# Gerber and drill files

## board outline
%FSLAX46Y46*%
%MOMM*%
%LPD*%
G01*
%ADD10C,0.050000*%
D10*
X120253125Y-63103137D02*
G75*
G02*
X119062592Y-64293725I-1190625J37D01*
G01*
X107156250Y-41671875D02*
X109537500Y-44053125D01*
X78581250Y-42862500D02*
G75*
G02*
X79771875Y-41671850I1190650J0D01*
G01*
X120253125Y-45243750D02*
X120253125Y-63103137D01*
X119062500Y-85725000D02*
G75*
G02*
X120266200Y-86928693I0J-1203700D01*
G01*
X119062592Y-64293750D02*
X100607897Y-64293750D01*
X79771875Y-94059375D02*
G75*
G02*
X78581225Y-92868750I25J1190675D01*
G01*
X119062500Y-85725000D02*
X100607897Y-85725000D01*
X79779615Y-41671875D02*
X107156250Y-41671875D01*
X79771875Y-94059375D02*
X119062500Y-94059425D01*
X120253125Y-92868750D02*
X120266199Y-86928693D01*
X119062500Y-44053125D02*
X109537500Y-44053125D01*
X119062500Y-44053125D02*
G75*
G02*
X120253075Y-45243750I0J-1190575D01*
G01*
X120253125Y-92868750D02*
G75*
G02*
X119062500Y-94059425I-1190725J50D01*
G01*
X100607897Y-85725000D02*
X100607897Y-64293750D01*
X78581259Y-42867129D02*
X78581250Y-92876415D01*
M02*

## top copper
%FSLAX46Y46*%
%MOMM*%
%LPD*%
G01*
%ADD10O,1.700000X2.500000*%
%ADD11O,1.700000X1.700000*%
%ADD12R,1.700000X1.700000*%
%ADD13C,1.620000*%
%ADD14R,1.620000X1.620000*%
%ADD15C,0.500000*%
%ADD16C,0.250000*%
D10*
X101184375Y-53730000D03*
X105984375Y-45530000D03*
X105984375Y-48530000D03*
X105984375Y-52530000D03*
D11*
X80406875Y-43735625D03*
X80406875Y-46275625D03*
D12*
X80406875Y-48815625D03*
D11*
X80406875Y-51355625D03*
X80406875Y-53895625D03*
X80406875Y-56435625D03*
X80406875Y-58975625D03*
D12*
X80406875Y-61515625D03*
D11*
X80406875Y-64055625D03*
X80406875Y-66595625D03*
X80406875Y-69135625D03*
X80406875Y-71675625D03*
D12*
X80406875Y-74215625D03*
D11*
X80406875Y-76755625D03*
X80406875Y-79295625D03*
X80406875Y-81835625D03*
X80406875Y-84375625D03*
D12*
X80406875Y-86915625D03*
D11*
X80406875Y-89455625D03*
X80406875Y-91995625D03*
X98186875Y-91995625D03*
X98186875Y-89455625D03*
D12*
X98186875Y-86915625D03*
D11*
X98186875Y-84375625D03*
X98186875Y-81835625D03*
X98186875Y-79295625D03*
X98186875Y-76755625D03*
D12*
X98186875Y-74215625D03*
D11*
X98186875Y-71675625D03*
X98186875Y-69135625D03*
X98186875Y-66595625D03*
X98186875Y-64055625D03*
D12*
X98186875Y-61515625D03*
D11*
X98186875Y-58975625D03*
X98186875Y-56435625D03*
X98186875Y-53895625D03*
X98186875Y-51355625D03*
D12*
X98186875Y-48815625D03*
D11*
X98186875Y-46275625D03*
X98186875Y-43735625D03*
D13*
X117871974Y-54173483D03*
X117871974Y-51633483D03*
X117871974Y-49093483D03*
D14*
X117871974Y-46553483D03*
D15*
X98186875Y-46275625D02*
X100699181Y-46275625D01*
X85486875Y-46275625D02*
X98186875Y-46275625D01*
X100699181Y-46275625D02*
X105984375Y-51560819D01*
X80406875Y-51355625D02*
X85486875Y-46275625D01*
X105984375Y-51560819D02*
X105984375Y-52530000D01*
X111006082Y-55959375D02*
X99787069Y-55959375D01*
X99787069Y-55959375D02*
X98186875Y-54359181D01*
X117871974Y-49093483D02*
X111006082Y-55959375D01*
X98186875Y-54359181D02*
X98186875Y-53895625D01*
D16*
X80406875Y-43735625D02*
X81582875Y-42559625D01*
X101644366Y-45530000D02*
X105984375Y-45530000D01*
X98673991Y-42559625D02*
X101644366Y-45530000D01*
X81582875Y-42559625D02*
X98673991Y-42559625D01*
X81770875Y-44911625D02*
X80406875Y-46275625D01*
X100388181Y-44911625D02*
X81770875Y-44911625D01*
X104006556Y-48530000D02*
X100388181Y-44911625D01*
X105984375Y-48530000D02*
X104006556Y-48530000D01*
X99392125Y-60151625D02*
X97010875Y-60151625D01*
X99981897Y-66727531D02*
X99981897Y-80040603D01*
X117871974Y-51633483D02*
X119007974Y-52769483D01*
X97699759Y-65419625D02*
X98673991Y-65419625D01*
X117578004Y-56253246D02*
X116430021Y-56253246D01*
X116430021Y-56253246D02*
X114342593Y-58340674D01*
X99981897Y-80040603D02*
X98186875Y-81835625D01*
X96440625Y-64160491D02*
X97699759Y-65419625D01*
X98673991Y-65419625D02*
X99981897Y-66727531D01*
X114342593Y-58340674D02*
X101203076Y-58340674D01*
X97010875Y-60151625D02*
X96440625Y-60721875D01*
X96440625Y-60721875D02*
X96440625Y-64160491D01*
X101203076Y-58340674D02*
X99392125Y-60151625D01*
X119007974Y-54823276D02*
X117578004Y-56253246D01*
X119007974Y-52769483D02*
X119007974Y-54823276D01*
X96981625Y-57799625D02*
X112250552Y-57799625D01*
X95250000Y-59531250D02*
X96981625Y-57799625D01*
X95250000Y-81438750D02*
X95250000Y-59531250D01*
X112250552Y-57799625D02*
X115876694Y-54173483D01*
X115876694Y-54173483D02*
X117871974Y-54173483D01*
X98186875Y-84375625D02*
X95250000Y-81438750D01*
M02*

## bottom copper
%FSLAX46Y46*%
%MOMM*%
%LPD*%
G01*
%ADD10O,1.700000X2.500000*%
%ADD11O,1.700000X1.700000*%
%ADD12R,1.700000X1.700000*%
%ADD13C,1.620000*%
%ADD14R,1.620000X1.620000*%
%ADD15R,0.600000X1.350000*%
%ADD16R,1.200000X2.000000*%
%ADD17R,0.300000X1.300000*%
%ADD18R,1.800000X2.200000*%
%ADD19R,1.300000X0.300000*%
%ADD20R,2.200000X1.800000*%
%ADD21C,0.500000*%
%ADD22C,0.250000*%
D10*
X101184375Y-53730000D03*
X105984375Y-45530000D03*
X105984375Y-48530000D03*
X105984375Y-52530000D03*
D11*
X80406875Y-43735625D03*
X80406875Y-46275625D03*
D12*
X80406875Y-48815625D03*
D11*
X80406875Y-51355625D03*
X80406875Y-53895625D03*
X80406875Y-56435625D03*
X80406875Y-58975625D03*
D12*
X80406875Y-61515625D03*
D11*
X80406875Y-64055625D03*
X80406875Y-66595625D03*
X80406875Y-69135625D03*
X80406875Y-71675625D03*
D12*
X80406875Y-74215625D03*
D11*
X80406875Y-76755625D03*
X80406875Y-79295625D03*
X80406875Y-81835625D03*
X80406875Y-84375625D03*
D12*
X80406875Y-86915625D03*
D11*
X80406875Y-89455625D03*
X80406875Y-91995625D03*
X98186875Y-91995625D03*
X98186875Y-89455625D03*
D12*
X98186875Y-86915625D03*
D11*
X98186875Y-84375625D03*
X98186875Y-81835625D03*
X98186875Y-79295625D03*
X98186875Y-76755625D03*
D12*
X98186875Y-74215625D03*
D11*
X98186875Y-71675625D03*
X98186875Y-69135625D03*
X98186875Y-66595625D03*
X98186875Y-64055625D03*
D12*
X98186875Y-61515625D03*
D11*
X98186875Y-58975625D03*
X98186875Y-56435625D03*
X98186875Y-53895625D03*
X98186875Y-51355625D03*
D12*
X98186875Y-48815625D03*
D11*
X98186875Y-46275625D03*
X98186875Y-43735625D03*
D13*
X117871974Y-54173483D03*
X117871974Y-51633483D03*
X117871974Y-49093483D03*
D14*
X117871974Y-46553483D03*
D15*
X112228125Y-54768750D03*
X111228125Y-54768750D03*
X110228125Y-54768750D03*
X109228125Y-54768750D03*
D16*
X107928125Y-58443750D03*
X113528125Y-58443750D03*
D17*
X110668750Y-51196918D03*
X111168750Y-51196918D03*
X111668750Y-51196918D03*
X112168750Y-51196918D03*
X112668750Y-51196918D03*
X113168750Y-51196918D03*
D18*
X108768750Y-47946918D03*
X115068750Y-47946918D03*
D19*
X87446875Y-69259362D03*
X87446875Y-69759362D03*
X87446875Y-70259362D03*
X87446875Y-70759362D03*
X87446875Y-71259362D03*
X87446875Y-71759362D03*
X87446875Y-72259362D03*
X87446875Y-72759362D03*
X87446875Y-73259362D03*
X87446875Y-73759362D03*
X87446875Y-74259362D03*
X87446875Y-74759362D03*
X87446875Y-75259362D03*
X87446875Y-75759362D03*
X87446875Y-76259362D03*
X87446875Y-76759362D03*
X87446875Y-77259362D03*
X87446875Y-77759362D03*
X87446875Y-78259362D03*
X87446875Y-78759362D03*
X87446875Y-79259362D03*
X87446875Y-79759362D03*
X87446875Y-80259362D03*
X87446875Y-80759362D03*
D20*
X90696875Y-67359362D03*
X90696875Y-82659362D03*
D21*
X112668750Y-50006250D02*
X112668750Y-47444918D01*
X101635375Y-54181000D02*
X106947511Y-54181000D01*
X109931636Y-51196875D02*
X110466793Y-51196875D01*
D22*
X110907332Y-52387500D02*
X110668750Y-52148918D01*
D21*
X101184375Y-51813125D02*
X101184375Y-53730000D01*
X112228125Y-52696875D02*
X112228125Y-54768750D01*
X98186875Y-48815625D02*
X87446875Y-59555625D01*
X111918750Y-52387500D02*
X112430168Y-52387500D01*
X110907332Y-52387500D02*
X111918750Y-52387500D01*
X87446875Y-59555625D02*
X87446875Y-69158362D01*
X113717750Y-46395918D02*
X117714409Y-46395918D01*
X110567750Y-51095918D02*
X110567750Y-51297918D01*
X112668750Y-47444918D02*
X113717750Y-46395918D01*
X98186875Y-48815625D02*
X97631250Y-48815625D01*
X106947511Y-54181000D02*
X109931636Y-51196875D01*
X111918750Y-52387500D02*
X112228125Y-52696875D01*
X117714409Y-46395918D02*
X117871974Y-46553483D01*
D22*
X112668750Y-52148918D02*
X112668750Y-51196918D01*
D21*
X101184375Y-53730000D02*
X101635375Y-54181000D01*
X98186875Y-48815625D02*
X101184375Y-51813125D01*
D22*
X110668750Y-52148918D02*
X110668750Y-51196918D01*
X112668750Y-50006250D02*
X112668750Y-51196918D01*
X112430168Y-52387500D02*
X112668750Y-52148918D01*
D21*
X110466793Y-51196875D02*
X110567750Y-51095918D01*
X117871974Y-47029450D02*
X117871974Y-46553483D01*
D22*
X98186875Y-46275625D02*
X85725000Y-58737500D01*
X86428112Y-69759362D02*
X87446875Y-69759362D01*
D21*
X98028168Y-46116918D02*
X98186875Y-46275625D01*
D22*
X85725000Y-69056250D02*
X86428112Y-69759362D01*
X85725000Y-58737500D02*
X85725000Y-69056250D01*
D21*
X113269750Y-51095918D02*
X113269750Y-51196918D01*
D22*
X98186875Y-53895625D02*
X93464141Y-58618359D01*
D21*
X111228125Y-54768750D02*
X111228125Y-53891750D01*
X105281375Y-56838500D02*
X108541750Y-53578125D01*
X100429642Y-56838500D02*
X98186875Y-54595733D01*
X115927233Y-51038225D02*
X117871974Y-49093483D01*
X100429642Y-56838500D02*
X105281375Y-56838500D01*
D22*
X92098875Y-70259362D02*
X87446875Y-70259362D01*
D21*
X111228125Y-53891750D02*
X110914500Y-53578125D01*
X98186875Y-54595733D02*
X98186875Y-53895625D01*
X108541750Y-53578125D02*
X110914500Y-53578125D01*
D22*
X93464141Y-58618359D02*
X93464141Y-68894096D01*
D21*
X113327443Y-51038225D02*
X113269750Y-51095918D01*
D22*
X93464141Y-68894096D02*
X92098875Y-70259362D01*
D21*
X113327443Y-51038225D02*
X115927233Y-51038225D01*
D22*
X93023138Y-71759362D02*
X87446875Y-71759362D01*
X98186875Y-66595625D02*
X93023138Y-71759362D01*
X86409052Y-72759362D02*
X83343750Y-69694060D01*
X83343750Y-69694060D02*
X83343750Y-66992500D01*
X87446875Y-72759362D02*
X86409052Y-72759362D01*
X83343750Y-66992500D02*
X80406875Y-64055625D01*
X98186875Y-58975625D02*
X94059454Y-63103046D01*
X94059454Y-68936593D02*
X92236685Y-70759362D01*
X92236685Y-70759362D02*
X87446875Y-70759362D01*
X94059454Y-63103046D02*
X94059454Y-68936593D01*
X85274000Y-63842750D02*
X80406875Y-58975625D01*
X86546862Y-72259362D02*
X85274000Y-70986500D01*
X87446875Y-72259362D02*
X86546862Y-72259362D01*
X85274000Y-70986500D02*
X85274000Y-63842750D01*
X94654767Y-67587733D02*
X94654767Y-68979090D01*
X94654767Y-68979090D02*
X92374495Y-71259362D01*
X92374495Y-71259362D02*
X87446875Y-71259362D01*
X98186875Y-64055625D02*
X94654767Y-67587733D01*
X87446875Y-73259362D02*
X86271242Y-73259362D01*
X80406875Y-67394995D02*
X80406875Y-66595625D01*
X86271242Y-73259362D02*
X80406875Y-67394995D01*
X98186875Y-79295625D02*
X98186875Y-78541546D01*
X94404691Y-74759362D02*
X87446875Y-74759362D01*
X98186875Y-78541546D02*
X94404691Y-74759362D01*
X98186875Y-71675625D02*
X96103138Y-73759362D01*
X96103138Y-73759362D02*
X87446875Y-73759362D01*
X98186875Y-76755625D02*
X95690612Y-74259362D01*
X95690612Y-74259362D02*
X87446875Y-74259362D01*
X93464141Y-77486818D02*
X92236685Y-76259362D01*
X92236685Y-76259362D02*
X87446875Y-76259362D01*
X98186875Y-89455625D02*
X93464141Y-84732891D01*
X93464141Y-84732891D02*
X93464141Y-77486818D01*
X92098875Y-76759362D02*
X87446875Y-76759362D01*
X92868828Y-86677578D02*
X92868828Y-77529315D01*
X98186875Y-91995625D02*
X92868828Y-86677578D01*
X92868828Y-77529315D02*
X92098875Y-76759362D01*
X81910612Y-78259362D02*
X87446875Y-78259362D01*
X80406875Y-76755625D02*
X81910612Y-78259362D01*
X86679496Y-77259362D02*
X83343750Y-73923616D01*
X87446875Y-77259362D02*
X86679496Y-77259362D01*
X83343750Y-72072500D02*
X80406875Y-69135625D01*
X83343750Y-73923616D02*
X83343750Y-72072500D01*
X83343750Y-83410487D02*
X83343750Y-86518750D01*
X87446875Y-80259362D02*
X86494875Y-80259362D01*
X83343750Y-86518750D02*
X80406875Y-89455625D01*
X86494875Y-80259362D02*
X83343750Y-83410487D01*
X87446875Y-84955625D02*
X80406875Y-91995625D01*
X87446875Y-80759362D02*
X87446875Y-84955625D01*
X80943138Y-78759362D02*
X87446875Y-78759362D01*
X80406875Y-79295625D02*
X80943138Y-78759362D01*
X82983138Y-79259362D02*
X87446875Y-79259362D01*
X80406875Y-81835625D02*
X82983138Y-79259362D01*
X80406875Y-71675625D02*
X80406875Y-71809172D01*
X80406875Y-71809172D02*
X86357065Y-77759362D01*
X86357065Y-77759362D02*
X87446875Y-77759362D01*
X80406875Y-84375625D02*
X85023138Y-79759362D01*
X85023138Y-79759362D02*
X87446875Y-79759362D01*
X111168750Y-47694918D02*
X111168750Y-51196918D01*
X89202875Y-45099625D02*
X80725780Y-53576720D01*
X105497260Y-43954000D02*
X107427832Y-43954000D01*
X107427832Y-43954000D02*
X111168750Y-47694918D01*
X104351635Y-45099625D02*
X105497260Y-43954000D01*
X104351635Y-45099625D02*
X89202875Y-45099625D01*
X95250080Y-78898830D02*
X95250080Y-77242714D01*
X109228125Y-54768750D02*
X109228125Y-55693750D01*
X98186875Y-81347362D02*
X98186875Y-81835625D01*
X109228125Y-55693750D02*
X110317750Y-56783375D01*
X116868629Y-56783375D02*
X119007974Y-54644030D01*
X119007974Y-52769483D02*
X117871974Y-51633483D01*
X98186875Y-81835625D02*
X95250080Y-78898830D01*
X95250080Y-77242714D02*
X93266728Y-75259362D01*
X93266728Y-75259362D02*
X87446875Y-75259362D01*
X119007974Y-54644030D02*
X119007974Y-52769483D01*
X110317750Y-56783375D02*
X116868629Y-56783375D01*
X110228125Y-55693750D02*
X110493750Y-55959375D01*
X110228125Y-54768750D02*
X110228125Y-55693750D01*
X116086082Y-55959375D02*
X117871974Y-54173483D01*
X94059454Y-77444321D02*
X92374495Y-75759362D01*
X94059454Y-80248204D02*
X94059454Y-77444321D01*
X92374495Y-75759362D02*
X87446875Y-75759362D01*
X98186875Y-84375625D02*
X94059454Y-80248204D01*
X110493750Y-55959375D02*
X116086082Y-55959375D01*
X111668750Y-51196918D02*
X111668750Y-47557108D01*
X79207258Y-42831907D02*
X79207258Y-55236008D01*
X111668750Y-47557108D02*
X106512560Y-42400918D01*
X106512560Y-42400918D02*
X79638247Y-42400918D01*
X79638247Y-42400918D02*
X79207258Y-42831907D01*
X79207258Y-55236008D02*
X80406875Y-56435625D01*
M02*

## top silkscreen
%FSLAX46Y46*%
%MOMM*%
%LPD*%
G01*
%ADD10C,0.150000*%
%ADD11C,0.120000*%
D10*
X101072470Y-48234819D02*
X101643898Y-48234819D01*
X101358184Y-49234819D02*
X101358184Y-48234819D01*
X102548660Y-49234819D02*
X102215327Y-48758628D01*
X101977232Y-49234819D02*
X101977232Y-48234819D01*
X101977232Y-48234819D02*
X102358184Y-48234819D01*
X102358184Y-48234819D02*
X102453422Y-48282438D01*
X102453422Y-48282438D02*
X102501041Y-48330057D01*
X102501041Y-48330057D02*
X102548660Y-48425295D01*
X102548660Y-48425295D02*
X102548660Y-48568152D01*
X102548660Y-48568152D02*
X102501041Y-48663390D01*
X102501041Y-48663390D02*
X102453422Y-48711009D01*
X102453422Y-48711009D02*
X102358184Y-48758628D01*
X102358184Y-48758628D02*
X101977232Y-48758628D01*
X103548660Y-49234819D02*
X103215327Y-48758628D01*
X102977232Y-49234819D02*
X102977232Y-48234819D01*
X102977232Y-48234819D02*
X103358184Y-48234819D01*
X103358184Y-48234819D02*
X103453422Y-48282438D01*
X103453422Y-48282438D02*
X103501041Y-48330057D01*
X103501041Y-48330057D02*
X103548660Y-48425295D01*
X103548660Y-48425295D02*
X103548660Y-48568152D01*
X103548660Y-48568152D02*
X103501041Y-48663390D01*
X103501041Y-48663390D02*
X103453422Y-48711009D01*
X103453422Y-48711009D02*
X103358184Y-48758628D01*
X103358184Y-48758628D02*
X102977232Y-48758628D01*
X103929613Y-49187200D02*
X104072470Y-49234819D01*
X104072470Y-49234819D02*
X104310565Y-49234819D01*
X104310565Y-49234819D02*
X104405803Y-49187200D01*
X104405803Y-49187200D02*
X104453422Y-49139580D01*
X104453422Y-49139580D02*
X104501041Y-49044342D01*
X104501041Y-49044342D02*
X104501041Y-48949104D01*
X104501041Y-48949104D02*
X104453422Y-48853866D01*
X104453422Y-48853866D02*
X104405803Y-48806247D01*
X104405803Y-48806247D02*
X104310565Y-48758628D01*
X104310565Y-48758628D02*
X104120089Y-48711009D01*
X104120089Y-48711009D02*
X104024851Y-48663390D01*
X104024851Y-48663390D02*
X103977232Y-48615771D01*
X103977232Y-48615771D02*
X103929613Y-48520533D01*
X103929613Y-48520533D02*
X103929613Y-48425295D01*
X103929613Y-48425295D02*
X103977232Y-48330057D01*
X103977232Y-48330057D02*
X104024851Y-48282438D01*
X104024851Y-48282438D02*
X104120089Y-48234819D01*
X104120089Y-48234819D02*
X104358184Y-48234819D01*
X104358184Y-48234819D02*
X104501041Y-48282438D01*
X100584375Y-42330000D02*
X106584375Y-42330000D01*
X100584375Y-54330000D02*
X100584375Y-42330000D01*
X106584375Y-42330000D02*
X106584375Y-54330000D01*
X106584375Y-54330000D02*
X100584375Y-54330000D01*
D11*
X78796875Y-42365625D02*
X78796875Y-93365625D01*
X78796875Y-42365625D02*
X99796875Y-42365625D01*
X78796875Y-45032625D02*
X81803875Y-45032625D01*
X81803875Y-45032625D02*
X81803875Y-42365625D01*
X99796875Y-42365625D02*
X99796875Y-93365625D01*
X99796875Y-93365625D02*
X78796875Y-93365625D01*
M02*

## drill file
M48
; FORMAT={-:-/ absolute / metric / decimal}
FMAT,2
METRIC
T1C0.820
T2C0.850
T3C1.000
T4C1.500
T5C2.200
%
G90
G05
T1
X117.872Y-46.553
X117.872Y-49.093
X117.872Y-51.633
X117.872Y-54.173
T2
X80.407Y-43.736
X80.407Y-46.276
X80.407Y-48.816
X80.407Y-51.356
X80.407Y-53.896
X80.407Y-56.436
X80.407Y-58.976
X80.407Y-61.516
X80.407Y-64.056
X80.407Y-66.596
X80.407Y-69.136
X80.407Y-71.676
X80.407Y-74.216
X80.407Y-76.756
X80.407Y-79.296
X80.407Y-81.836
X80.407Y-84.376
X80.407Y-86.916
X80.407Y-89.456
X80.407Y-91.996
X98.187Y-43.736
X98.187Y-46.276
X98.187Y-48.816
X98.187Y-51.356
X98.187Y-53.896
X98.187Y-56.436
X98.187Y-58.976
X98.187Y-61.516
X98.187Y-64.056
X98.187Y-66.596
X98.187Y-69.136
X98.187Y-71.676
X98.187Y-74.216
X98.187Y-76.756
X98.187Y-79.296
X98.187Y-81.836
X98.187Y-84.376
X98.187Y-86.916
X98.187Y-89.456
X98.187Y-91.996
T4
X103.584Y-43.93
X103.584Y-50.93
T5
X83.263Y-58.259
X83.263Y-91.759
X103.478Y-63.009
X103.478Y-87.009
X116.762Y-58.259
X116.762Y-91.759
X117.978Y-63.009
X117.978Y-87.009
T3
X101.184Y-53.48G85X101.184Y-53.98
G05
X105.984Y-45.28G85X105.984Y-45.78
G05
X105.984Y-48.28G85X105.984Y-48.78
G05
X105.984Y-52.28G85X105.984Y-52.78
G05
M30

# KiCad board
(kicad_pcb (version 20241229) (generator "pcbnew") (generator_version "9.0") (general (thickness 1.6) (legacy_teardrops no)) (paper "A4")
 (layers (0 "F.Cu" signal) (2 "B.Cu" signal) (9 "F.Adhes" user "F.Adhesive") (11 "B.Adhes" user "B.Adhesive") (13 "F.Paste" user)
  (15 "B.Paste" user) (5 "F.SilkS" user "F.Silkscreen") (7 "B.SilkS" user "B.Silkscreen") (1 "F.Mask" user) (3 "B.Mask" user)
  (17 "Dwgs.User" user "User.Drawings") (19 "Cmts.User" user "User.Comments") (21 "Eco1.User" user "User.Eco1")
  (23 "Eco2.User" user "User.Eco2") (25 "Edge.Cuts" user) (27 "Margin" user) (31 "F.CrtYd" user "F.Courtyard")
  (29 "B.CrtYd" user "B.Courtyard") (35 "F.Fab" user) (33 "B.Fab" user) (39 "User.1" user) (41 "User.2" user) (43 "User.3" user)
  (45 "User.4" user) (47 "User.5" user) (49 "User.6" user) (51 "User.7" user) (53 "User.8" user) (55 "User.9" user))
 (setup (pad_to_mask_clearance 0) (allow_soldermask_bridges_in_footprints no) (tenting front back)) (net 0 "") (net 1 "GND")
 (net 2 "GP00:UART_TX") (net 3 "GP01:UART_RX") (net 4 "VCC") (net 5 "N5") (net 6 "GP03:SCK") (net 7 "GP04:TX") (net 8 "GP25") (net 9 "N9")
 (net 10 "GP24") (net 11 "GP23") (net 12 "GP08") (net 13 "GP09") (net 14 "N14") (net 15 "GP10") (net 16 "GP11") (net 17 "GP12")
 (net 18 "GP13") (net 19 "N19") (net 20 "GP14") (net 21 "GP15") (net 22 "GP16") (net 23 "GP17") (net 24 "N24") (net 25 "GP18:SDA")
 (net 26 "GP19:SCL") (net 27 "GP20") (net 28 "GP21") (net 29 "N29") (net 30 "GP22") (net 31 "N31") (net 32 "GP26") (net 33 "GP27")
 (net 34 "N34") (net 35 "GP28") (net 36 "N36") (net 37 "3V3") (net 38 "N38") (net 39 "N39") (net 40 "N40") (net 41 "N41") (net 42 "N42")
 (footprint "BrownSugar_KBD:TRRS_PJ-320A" (layer "F.Cu") (at 103.584375 42.33)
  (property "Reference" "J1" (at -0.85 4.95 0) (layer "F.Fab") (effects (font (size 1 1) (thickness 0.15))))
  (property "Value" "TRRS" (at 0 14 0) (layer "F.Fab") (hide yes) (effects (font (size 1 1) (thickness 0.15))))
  (fp_line (start -3 0) (end 3 0) (stroke (width 0.15) (type solid)) (layer "F.SilkS"))
  (fp_line (start -3 12) (end -3 0) (stroke (width 0.15) (type solid)) (layer "F.SilkS"))
  (fp_line (start 3 0) (end 3 12) (stroke (width 0.15) (type solid)) (layer "F.SilkS"))
  (fp_line (start 3 12) (end -3 12) (stroke (width 0.15) (type solid)) (layer "F.SilkS"))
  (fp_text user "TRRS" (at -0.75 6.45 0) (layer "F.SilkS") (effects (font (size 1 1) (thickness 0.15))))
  (pad "" np_thru_hole circle (at 0 1.6) (size 1.5 1.5) (drill 1.5) (layers "*.Cu" "*.Mask"))
  (pad "" np_thru_hole circle (at 0 8.6) (size 1.5 1.5) (drill 1.5) (layers "*.Cu" "*.Mask"))
  (pad "A" thru_hole oval (at -2.4 11.4) (size 1.7 2.5) (drill oval 1 1.5) (layers "*.Cu" "*.Mask") (remove_unused_layers no) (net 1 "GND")
   (clearance 0.15))
  (pad "B" thru_hole oval (at 2.4 3.2) (size 1.7 2.5) (drill oval 1 1.5) (layers "*.Cu" "*.Mask") (remove_unused_layers no)
   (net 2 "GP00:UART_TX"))
  (pad "C" thru_hole oval (at 2.4 6.2) (size 1.7 2.5) (drill oval 1 1.5) (layers "*.Cu" "*.Mask") (remove_unused_layers no)
   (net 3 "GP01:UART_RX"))
  (pad "D" thru_hole oval (at 2.4 10.2) (size 1.7 2.5) (drill oval 1 1.5) (layers "*.Cu" "*.Mask") (remove_unused_layers no) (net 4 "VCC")
   (clearance 0.15)))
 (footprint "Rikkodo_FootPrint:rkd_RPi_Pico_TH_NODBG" (layer "F.Cu") (at 89.296875 67.865625)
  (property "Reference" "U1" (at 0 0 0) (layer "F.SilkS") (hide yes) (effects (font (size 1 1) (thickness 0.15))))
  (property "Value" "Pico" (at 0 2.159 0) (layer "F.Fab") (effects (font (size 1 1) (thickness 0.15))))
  (fp_line (start -10.5 -25.5) (end -10.5 25.5) (stroke (width 0.12) (type solid)) (layer "F.SilkS"))
  (fp_line (start -10.5 -25.5) (end 10.5 -25.5) (stroke (width 0.12) (type solid)) (layer "F.SilkS"))
  (fp_line (start -10.5 -22.833) (end -7.493 -22.833) (stroke (width 0.12) (type solid)) (layer "F.SilkS"))
  (fp_line (start -7.493 -22.833) (end -7.493 -25.5) (stroke (width 0.12) (type solid)) (layer "F.SilkS"))
  (fp_line (start 10.5 -25.5) (end 10.5 25.5) (stroke (width 0.12) (type solid)) (layer "F.SilkS"))
  (fp_line (start 10.5 25.5) (end -10.5 25.5) (stroke (width 0.12) (type solid)) (layer "F.SilkS"))
  (pad "1" thru_hole oval (at -8.89 -24.13) (size 1.7 1.7) (drill 0.85) (layers "*.Cu" "*.Mask") (remove_unused_layers no)
   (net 2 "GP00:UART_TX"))
  (pad "2" thru_hole oval (at -8.89 -21.59) (size 1.7 1.7) (drill 0.85) (layers "*.Cu" "*.Mask") (remove_unused_layers no)
   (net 3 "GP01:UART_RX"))
  (pad "3" thru_hole rect (at -8.89 -19.05) (size 1.7 1.7) (drill 0.85) (layers "*.Cu" "*.Mask") (remove_unused_layers no) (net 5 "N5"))
  (pad "4" thru_hole oval (at -8.89 -16.51) (size 1.7 1.7) (drill 0.85) (layers "*.Cu" "*.Mask") (remove_unused_layers no) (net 4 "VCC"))
  (pad "5" thru_hole oval (at -8.89 -13.97) (size 1.7 1.7) (drill 0.85) (layers "*.Cu" "*.Mask") (remove_unused_layers no)
   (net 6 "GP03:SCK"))
  (pad "6" thru_hole oval (at -8.89 -11.43) (size 1.7 1.7) (drill 0.85) (layers "*.Cu" "*.Mask") (remove_unused_layers no) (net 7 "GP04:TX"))
  (pad "7" thru_hole oval (at -8.89 -8.89) (size 1.7 1.7) (drill 0.85) (layers "*.Cu" "*.Mask") (remove_unused_layers no) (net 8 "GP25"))
  (pad "8" thru_hole rect (at -8.89 -6.35) (size 1.7 1.7) (drill 0.85) (layers "*.Cu" "*.Mask") (remove_unused_layers no) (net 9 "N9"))
  (pad "9" thru_hole oval (at -8.89 -3.81) (size 1.7 1.7) (drill 0.85) (layers "*.Cu" "*.Mask") (remove_unused_layers no) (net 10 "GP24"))
  (pad "10" thru_hole oval (at -8.89 -1.27) (size 1.7 1.7) (drill 0.85) (layers "*.Cu" "*.Mask") (remove_unused_layers no) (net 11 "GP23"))
  (pad "11" thru_hole oval (at -8.89 1.27) (size 1.7 1.7) (drill 0.85) (layers "*.Cu" "*.Mask") (remove_unused_layers no) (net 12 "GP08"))
  (pad "12" thru_hole oval (at -8.89 3.81) (size 1.7 1.7) (drill 0.85) (layers "*.Cu" "*.Mask") (remove_unused_layers no) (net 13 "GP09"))
  (pad "13" thru_hole rect (at -8.89 6.35) (size 1.7 1.7) (drill 0.85) (layers "*.Cu" "*.Mask") (remove_unused_layers no) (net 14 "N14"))
  (pad "14" thru_hole oval (at -8.89 8.89) (size 1.7 1.7) (drill 0.85) (layers "*.Cu" "*.Mask") (remove_unused_layers no) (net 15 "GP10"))
  (pad "15" thru_hole oval (at -8.89 11.43) (size 1.7 1.7) (drill 0.85) (layers "*.Cu" "*.Mask") (remove_unused_layers no) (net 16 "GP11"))
  (pad "16" thru_hole oval (at -8.89 13.97) (size 1.7 1.7) (drill 0.85) (layers "*.Cu" "*.Mask") (remove_unused_layers no) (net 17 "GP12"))
  (pad "17" thru_hole oval (at -8.89 16.51) (size 1.7 1.7) (drill 0.85) (layers "*.Cu" "*.Mask") (remove_unused_layers no) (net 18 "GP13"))
  (pad "18" thru_hole rect (at -8.89 19.05) (size 1.7 1.7) (drill 0.85) (layers "*.Cu" "*.Mask") (remove_unused_layers no) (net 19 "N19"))
  (pad "19" thru_hole oval (at -8.89 21.59) (size 1.7 1.7) (drill 0.85) (layers "*.Cu" "*.Mask") (remove_unused_layers no) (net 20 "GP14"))
  (pad "20" thru_hole oval (at -8.89 24.13) (size 1.7 1.7) (drill 0.85) (layers "*.Cu" "*.Mask") (remove_unused_layers no) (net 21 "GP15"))
  (pad "21" thru_hole oval (at 8.89 24.13) (size 1.7 1.7) (drill 0.85) (layers "*.Cu" "*.Mask") (remove_unused_layers no) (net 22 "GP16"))
  (pad "22" thru_hole oval (at 8.89 21.59) (size 1.7 1.7) (drill 0.85) (layers "*.Cu" "*.Mask") (remove_unused_layers no) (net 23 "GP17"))
  (pad "23" thru_hole rect (at 8.89 19.05) (size 1.7 1.7) (drill 0.85) (layers "*.Cu" "*.Mask") (remove_unused_layers no) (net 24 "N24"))
  (pad "24" thru_hole oval (at 8.89 16.51) (size 1.7 1.7) (drill 0.85) (layers "*.Cu" "*.Mask") (remove_unused_layers no)
   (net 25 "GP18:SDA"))
  (pad "25" thru_hole oval (at 8.89 13.97) (size 1.7 1.7) (drill 0.85) (layers "*.Cu" "*.Mask") (remove_unused_layers no)
   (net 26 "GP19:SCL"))
  (pad "26" thru_hole oval (at 8.89 11.43) (size 1.7 1.7) (drill 0.85) (layers "*.Cu" "*.Mask") (remove_unused_layers no) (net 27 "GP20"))
  (pad "27" thru_hole oval (at 8.89 8.89) (size 1.7 1.7) (drill 0.85) (layers "*.Cu" "*.Mask") (remove_unused_layers no) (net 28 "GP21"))
  (pad "28" thru_hole rect (at 8.89 6.35) (size 1.7 1.7) (drill 0.85) (layers "*.Cu" "*.Mask") (remove_unused_layers no) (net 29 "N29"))
  (pad "29" thru_hole oval (at 8.89 3.81) (size 1.7 1.7) (drill 0.85) (layers "*.Cu" "*.Mask") (remove_unused_layers no) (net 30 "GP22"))
  (pad "30" thru_hole oval (at 8.89 1.27) (size 1.7 1.7) (drill 0.85) (layers "*.Cu" "*.Mask") (remove_unused_layers no) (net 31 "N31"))
  (pad "31" thru_hole oval (at 8.89 -1.27) (size 1.7 1.7) (drill 0.85) (layers "*.Cu" "*.Mask") (remove_unused_layers no) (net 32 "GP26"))
  (pad "32" thru_hole oval (at 8.89 -3.81) (size 1.7 1.7) (drill 0.85) (layers "*.Cu" "*.Mask") (remove_unused_layers no) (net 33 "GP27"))
  (pad "33" thru_hole rect (at 8.89 -6.35) (size 1.7 1.7) (drill 0.85) (layers "*.Cu" "*.Mask") (remove_unused_layers no) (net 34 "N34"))
  (pad "34" thru_hole oval (at 8.89 -8.89) (size 1.7 1.7) (drill 0.85) (layers "*.Cu" "*.Mask") (remove_unused_layers no) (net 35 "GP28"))
  (pad "35" thru_hole oval (at 8.89 -11.43) (size 1.7 1.7) (drill 0.85) (layers "*.Cu" "*.Mask") (remove_unused_layers no) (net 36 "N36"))
  (pad "36" thru_hole oval (at 8.89 -13.97) (size 1.7 1.7) (drill 0.85) (layers "*.Cu" "*.Mask") (remove_unused_layers no) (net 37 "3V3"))
  (pad "37" thru_hole oval (at 8.89 -16.51) (size 1.7 1.7) (drill 0.85) (layers "*.Cu" "*.Mask") (remove_unused_layers no) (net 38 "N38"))
  (pad "38" thru_hole rect (at 8.89 -19.05) (size 1.7 1.7) (drill 0.85) (layers "*.Cu" "*.Mask") (remove_unused_layers no) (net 1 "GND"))
  (pad "39" thru_hole oval (at 8.89 -21.59) (size 1.7 1.7) (drill 0.85) (layers "*.Cu" "*.Mask") (remove_unused_layers no) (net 4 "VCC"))
  (pad "40" thru_hole oval (at 8.89 -24.13) (size 1.7 1.7) (drill 0.85) (layers "*.Cu" "*.Mask") (remove_unused_layers no) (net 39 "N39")))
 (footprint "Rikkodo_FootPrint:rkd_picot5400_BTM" (layer "F.Cu") (at 100.0125 75.009375)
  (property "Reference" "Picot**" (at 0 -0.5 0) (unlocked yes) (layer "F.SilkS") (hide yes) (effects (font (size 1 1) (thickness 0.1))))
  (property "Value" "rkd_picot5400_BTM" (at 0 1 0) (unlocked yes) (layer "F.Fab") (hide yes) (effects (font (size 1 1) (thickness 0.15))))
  (pad "" np_thru_hole circle (at -16.75 -16.75) (size 2.2 2.2) (drill 2.2) (layers "*.Cu" "*.Mask"))
  (pad "" np_thru_hole circle (at -16.75 16.75) (size 2.2 2.2) (drill 2.2) (layers "*.Cu" "*.Mask"))
  (pad "" np_thru_hole circle (at 16.75 -16.75) (size 2.2 2.2) (drill 2.2) (layers "*.Cu" "*.Mask"))
  (pad "" np_thru_hole circle (at 16.75 16.75) (size 2.2 2.2) (drill 2.2) (layers "*.Cu" "*.Mask")))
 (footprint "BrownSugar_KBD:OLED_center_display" (layer "F.Cu") (at 99.371974 50.363483 90)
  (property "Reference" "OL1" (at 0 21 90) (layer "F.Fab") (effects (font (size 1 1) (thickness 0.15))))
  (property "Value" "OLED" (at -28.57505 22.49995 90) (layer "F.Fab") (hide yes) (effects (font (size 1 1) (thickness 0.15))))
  (pad "1" thru_hole circle (at -3.81 18.5 90) (size 1.62 1.62) (drill 0.82) (layers "*.Cu" "*.Mask") (remove_unused_layers no)
   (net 25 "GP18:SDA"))
  (pad "2" thru_hole circle (at -1.27 18.5 90) (size 1.62 1.62) (drill 0.82) (layers "*.Cu" "*.Mask") (remove_unused_layers no)
   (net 26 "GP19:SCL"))
  (pad "3" thru_hole circle (at 1.27 18.5 90) (size 1.62 1.62) (drill 0.82) (layers "*.Cu" "*.Mask") (remove_unused_layers no)
   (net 37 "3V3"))
  (pad "4" thru_hole rect (at 3.81 18.5 90) (size 1.62 1.62) (drill 0.82) (layers "*.Cu" "*.Mask") (remove_unused_layers no) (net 1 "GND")))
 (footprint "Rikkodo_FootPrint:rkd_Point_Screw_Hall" (layer "F.Cu") (at 110.728125 75.009375)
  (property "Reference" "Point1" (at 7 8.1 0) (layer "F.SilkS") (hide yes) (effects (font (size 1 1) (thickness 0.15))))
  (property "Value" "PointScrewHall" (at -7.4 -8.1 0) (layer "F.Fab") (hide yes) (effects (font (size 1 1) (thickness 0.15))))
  (pad "" np_thru_hole circle (at -7.25 -12) (size 2.2 2.2) (drill 2.2) (layers "*.Cu" "*.Mask"))
  (pad "" np_thru_hole circle (at -7.25 12) (size 2.2 2.2) (drill 2.2) (layers "*.Cu" "*.Mask"))
  (pad "" np_thru_hole circle (at 7.25 -12) (size 2.2 2.2) (drill 2.2) (layers "*.Cu" "*.Mask"))
  (pad "" np_thru_hole circle (at 7.25 12) (size 2.2 2.2) (drill 2.2) (layers "*.Cu" "*.Mask")))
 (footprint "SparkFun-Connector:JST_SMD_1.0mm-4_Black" (layer "B.Cu") (at 110.728125 54.76875 180)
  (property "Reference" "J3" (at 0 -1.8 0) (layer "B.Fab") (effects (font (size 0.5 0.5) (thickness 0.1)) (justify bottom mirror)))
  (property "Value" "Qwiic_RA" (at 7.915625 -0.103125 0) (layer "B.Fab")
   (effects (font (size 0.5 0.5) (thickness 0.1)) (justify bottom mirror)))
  (pad "1" smd rect (at -1.5 0 180) (size 0.6 1.35) (layers "B.Cu" "B.Mask" "B.Paste") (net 1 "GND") (thermal_bridge_angle 0))
  (pad "2" smd rect (at -0.5 0 180) (size 0.6 1.35) (layers "B.Cu" "B.Mask" "B.Paste") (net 37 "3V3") (thermal_bridge_angle 0))
  (pad "3" smd rect (at 0.5 0 180) (size 0.6 1.35) (layers "B.Cu" "B.Mask" "B.Paste") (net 25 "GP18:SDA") (thermal_bridge_angle 0))
  (pad "4" smd rect (at 1.5 0 180) (size 0.6 1.35) (layers "B.Cu" "B.Mask" "B.Paste") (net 26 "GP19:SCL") (thermal_bridge_angle 0))
  (pad "NC1" smd rect (at 2.8 -3.675 180) (size 1.2 2) (layers "B.Cu" "B.Mask" "B.Paste") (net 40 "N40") (thermal_bridge_angle 0))
  (pad "NC2" smd rect (at -2.8 -3.675 180) (size 1.2 2) (layers "B.Cu" "B.Mask" "B.Paste") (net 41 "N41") (thermal_bridge_angle 0)))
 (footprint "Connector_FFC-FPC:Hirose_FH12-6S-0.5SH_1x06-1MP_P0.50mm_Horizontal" (layer "B.Cu") (at 111.91875 49.346918)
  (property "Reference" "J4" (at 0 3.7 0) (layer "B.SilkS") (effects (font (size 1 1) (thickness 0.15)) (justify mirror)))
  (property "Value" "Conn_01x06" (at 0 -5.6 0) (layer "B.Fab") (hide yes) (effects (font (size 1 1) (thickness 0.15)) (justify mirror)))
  (pad "1" smd rect (at -1.25 1.85) (size 0.3 1.3) (layers "B.Cu" "B.Mask" "B.Paste") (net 1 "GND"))
  (pad "2" smd rect (at -0.75 1.85) (size 0.3 1.3) (layers "B.Cu" "B.Mask" "B.Paste") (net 6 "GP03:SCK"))
  (pad "3" smd rect (at -0.25 1.85) (size 0.3 1.3) (layers "B.Cu" "B.Mask" "B.Paste") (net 7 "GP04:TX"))
  (pad "4" smd rect (at 0.25 1.85) (size 0.3 1.3) (layers "B.Cu" "B.Mask" "B.Paste") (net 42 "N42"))
  (pad "5" smd rect (at 0.75 1.85) (size 0.3 1.3) (layers "B.Cu" "B.Mask" "B.Paste") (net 1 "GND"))
  (pad "6" smd rect (at 1.25 1.85) (size 0.3 1.3) (layers "B.Cu" "B.Mask" "B.Paste") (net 37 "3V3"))
  (pad "MP" smd rect (at -3.15 -1.4) (size 1.8 2.2) (layers "B.Cu" "B.Mask" "B.Paste"))
  (pad "MP" smd rect (at 3.15 -1.4) (size 1.8 2.2) (layers "B.Cu" "B.Mask" "B.Paste")))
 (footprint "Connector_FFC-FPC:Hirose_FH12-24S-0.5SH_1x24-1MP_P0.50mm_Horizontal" (layer "B.Cu") (at 89.296875 75.009362 -90)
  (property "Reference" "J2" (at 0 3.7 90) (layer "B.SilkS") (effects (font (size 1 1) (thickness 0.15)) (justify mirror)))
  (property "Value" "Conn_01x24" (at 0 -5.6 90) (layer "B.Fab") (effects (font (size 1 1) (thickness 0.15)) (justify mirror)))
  (pad "1" smd rect (at -5.75 1.85 270) (size 0.3 1.3) (layers "B.Cu" "B.Mask" "B.Paste") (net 1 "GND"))
  (pad "2" smd rect (at -5.25 1.85 270) (size 0.3 1.3) (layers "B.Cu" "B.Mask" "B.Paste") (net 4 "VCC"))
  (pad "3" smd rect (at -4.75 1.85 270) (size 0.3 1.3) (layers "B.Cu" "B.Mask" "B.Paste") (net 37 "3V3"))
  (pad "4" smd rect (at -4.25 1.85 270) (size 0.3 1.3) (layers "B.Cu" "B.Mask" "B.Paste") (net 35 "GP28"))
  (pad "5" smd rect (at -3.75 1.85 270) (size 0.3 1.3) (layers "B.Cu" "B.Mask" "B.Paste") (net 33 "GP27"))
  (pad "6" smd rect (at -3.25 1.85 270) (size 0.3 1.3) (layers "B.Cu" "B.Mask" "B.Paste") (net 32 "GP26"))
  (pad "7" smd rect (at -2.75 1.85 270) (size 0.3 1.3) (layers "B.Cu" "B.Mask" "B.Paste") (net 8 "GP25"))
  (pad "8" smd rect (at -2.25 1.85 270) (size 0.3 1.3) (layers "B.Cu" "B.Mask" "B.Paste") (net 10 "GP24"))
  (pad "9" smd rect (at -1.75 1.85 270) (size 0.3 1.3) (layers "B.Cu" "B.Mask" "B.Paste") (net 11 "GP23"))
  (pad "10" smd rect (at -1.25 1.85 270) (size 0.3 1.3) (layers "B.Cu" "B.Mask" "B.Paste") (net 30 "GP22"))
  (pad "11" smd rect (at -0.75 1.85 270) (size 0.3 1.3) (layers "B.Cu" "B.Mask" "B.Paste") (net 28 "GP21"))
  (pad "12" smd rect (at -0.25 1.85 270) (size 0.3 1.3) (layers "B.Cu" "B.Mask" "B.Paste") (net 27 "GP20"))
  (pad "13" smd rect (at 0.25 1.85 270) (size 0.3 1.3) (layers "B.Cu" "B.Mask" "B.Paste") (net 26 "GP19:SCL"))
  (pad "14" smd rect (at 0.75 1.85 270) (size 0.3 1.3) (layers "B.Cu" "B.Mask" "B.Paste") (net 25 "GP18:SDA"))
  (pad "15" smd rect (at 1.25 1.85 270) (size 0.3 1.3) (layers "B.Cu" "B.Mask" "B.Paste") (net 23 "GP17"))
  (pad "16" smd rect (at 1.75 1.85 270) (size 0.3 1.3) (layers "B.Cu" "B.Mask" "B.Paste") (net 22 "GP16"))
  (pad "17" smd rect (at 2.25 1.85 270) (size 0.3 1.3) (layers "B.Cu" "B.Mask" "B.Paste") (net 12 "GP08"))
  (pad "18" smd rect (at 2.75 1.85 270) (size 0.3 1.3) (layers "B.Cu" "B.Mask" "B.Paste") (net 13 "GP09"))
  (pad "19" smd rect (at 3.25 1.85 270) (size 0.3 1.3) (layers "B.Cu" "B.Mask" "B.Paste") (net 15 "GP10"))
  (pad "20" smd rect (at 3.75 1.85 270) (size 0.3 1.3) (layers "B.Cu" "B.Mask" "B.Paste") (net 16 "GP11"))
  (pad "21" smd rect (at 4.25 1.85 270) (size 0.3 1.3) (layers "B.Cu" "B.Mask" "B.Paste") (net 17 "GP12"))
  (pad "22" smd rect (at 4.75 1.85 270) (size 0.3 1.3) (layers "B.Cu" "B.Mask" "B.Paste") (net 18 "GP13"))
  (pad "23" smd rect (at 5.25 1.85 270) (size 0.3 1.3) (layers "B.Cu" "B.Mask" "B.Paste") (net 20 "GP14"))
  (pad "24" smd rect (at 5.75 1.85 270) (size 0.3 1.3) (layers "B.Cu" "B.Mask" "B.Paste") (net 21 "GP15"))
  (pad "MP" smd rect (at -7.65 -1.4 270) (size 1.8 2.2) (layers "B.Cu" "B.Mask" "B.Paste"))
  (pad "MP" smd rect (at 7.65 -1.4 270) (size 1.8 2.2) (layers "B.Cu" "B.Mask" "B.Paste")))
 (gr_arc (start 120.253125 63.103137) (mid 119.904427 63.944996) (end 119.062592 64.29375) (stroke (width 0.05) (type default))
  (layer "Edge.Cuts"))
 (gr_line (start 107.15625 41.671875) (end 109.5375 44.053125) (stroke (width 0.05) (type default)) (layer "Edge.Cuts"))
 (gr_arc (start 78.58125 42.8625) (mid 78.929974 42.020592) (end 79.771875 41.671875) (stroke (width 0.05) (type default))
  (layer "Edge.Cuts"))
 (gr_line (start 120.253125 45.24375) (end 120.253125 63.103137) (stroke (width 0.05) (type default)) (layer "Edge.Cuts"))
 (gr_arc (start 119.0625 85.725) (mid 119.913639 86.077554) (end 120.266193 86.928693) (stroke (width 0.05) (type default))
  (layer "Edge.Cuts"))
 (gr_line (start 119.062592 64.29375) (end 100.607897 64.29375) (stroke (width 0.05) (type default)) (layer "Edge.Cuts"))
 (gr_arc (start 79.771875 94.059375) (mid 78.929974 93.710643) (end 78.58125 92.86875) (stroke (width 0.05) (type default))
  (layer "Edge.Cuts"))
 (gr_line (start 119.0625 85.725) (end 100.607897 85.725) (stroke (width 0.05) (type default)) (layer "Edge.Cuts"))
 (gr_line (start 79.779615 41.671875) (end 107.15625 41.671875) (stroke (width 0.05) (type default)) (layer "Edge.Cuts"))
 (gr_line (start 79.771875 94.059375) (end 119.0625 94.059425) (stroke (width 0.05) (type default)) (layer "Edge.Cuts"))
 (gr_line (start 120.253125 92.86875) (end 120.266199 86.928693) (stroke (width 0.05) (type default)) (layer "Edge.Cuts"))
 (gr_line (start 119.0625 44.053125) (end 109.5375 44.053125) (stroke (width 0.05) (type default)) (layer "Edge.Cuts"))
 (gr_arc (start 119.0625 44.053125) (mid 119.904417 44.401848) (end 120.253125 45.24375) (stroke (width 0.05) (type default))
  (layer "Edge.Cuts"))
 (gr_arc (start 120.253125 92.86875) (mid 119.904381 93.710617) (end 119.0625 94.059375) (stroke (width 0.05) (type default))
  (layer "Edge.Cuts"))
 (gr_line (start 100.607897 85.725) (end 100.607897 64.29375) (stroke (width 0.05) (type default)) (layer "Edge.Cuts"))
 (gr_line (start 78.581259 42.867129) (end 78.58125 92.876415) (stroke (width 0.05) (type default)) (layer "Edge.Cuts"))
 (segment (start 112.66875 50.00625) (end 112.66875 47.444918) (width 0.5) (layer "B.Cu") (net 1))
 (segment (start 101.635375 54.181) (end 106.947511 54.181) (width 0.5) (layer "B.Cu") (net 1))
 (segment (start 109.931636 51.196875) (end 110.466793 51.196875) (width 0.5) (layer "B.Cu") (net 1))
 (segment (start 110.907332 52.3875) (end 110.66875 52.148918) (width 0.25) (layer "B.Cu") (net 1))
 (segment (start 101.184375 51.813125) (end 101.184375 53.73) (width 0.5) (layer "B.Cu") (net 1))
 (segment (start 112.228125 52.696875) (end 112.228125 54.76875) (width 0.5) (layer "B.Cu") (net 1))
 (segment (start 98.186875 48.815625) (end 87.446875 59.555625) (width 0.5) (layer "B.Cu") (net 1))
 (segment (start 111.91875 52.3875) (end 112.430168 52.3875) (width 0.5) (layer "B.Cu") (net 1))
 (segment (start 110.907332 52.3875) (end 111.91875 52.3875) (width 0.5) (layer "B.Cu") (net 1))
 (segment (start 87.446875 59.555625) (end 87.446875 69.158362) (width 0.5) (layer "B.Cu") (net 1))
 (segment (start 113.71775 46.395918) (end 117.714409 46.395918) (width 0.5) (layer "B.Cu") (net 1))
 (segment (start 110.56775 51.095918) (end 110.56775 51.297918) (width 0.5) (layer "B.Cu") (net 1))
 (segment (start 112.66875 47.444918) (end 113.71775 46.395918) (width 0.5) (layer "B.Cu") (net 1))
 (segment (start 98.186875 48.815625) (end 97.63125 48.815625) (width 0.5) (layer "B.Cu") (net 1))
 (segment (start 106.947511 54.181) (end 109.931636 51.196875) (width 0.5) (layer "B.Cu") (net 1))
 (segment (start 111.91875 52.3875) (end 112.228125 52.696875) (width 0.5) (layer "B.Cu") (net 1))
 (segment (start 117.714409 46.395918) (end 117.871974 46.553483) (width 0.5) (layer "B.Cu") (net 1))
 (segment (start 112.66875 52.148918) (end 112.66875 51.196918) (width 0.25) (layer "B.Cu") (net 1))
 (segment (start 101.184375 53.73) (end 101.635375 54.181) (width 0.5) (layer "B.Cu") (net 1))
 (segment (start 98.186875 48.815625) (end 101.184375 51.813125) (width 0.5) (layer "B.Cu") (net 1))
 (segment (start 110.66875 52.148918) (end 110.66875 51.196918) (width 0.25) (layer "B.Cu") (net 1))
 (segment (start 112.66875 50.00625) (end 112.66875 51.196918) (width 0.25) (layer "B.Cu") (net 1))
 (segment (start 112.430168 52.3875) (end 112.66875 52.148918) (width 0.25) (layer "B.Cu") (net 1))
 (segment (start 110.466793 51.196875) (end 110.56775 51.095918) (width 0.5) (layer "B.Cu") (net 1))
 (segment (start 117.871974 47.02945) (end 117.871974 46.553483) (width 0.5) (layer "B.Cu") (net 1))
 (segment (start 98.186875 46.275625) (end 100.699181 46.275625) (width 0.5) (layer "F.Cu") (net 4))
 (segment (start 85.486875 46.275625) (end 98.186875 46.275625) (width 0.5) (layer "F.Cu") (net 4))
 (segment (start 100.699181 46.275625) (end 105.984375 51.560819) (width 0.5) (layer "F.Cu") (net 4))
 (segment (start 80.406875 51.355625) (end 85.486875 46.275625) (width 0.5) (layer "F.Cu") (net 4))
 (segment (start 105.984375 51.560819) (end 105.984375 52.53) (width 0.5) (layer "F.Cu") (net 4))
 (segment (start 98.186875 46.275625) (end 85.725 58.7375) (width 0.25) (layer "B.Cu") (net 4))
 (segment (start 86.428112 69.759362) (end 87.446875 69.759362) (width 0.25) (layer "B.Cu") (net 4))
 (segment (start 98.028168 46.116918) (end 98.186875 46.275625) (width 0.5) (layer "B.Cu") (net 4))
 (segment (start 85.725 69.05625) (end 86.428112 69.759362) (width 0.25) (layer "B.Cu") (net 4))
 (segment (start 85.725 58.7375) (end 85.725 69.05625) (width 0.25) (layer "B.Cu") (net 4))
 (segment (start 111.006082 55.959375) (end 99.787069 55.959375) (width 0.5) (layer "F.Cu") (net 37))
 (segment (start 99.787069 55.959375) (end 98.186875 54.359181) (width 0.5) (layer "F.Cu") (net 37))
 (segment (start 117.871974 49.093483) (end 111.006082 55.959375) (width 0.5) (layer "F.Cu") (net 37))
 (segment (start 98.186875 54.359181) (end 98.186875 53.895625) (width 0.5) (layer "F.Cu") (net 37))
 (segment (start 113.26975 51.095918) (end 113.26975 51.196918) (width 0.5) (layer "B.Cu") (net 37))
 (segment (start 98.186875 53.895625) (end 93.464141 58.618359) (width 0.25) (layer "B.Cu") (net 37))
 (segment (start 111.228125 54.76875) (end 111.228125 53.89175) (width 0.5) (layer "B.Cu") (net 37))
 (segment (start 105.281375 56.8385) (end 108.54175 53.578125) (width 0.5) (layer "B.Cu") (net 37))
 (segment (start 100.429642 56.8385) (end 98.186875 54.595733) (width 0.5) (layer "B.Cu") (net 37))
 (segment (start 115.927233 51.038225) (end 117.871974 49.093483) (width 0.5) (layer "B.Cu") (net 37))
 (segment (start 100.429642 56.8385) (end 105.281375 56.8385) (width 0.5) (layer "B.Cu") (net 37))
 (segment (start 92.098875 70.259362) (end 87.446875 70.259362) (width 0.25) (layer "B.Cu") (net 37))
 (segment (start 111.228125 53.89175) (end 110.9145 53.578125) (width 0.5) (layer "B.Cu") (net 37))
 (segment (start 98.186875 54.595733) (end 98.186875 53.895625) (width 0.5) (layer "B.Cu") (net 37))
 (segment (start 108.54175 53.578125) (end 110.9145 53.578125) (width 0.5) (layer "B.Cu") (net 37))
 (segment (start 93.464141 58.618359) (end 93.464141 68.894096) (width 0.25) (layer "B.Cu") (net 37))
 (segment (start 113.327443 51.038225) (end 113.26975 51.095918) (width 0.5) (layer "B.Cu") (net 37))
 (segment (start 93.464141 68.894096) (end 92.098875 70.259362) (width 0.25) (layer "B.Cu") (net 37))
 (segment (start 113.327443 51.038225) (end 115.927233 51.038225) (width 0.5) (layer "B.Cu") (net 37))
 (segment (start 93.023138 71.759362) (end 87.446875 71.759362) (width 0.25) (layer "B.Cu") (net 32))
 (segment (start 98.186875 66.595625) (end 93.023138 71.759362) (width 0.25) (layer "B.Cu") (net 32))
 (segment (start 86.409052 72.759362) (end 83.34375 69.69406) (width 0.25) (layer "B.Cu") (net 10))
 (segment (start 83.34375 69.69406) (end 83.34375 66.9925) (width 0.25) (layer "B.Cu") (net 10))
 (segment (start 87.446875 72.759362) (end 86.409052 72.759362) (width 0.25) (layer "B.Cu") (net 10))
 (segment (start 83.34375 66.9925) (end 80.406875 64.055625) (width 0.25) (layer "B.Cu") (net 10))
 (segment (start 98.186875 58.975625) (end 94.059454 63.103046) (width 0.25) (layer "B.Cu") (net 35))
 (segment (start 94.059454 68.936593) (end 92.236685 70.759362) (width 0.25) (layer "B.Cu") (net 35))
 (segment (start 92.236685 70.759362) (end 87.446875 70.759362) (width 0.25) (layer "B.Cu") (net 35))
 (segment (start 94.059454 63.103046) (end 94.059454 68.936593) (width 0.25) (layer "B.Cu") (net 35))
 (segment (start 85.274 63.84275) (end 80.406875 58.975625) (width 0.25) (layer "B.Cu") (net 8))
 (segment (start 86.546862 72.259362) (end 85.274 70.9865) (width 0.25) (layer "B.Cu") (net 8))
 (segment (start 87.446875 72.259362) (end 86.546862 72.259362) (width 0.25) (layer "B.Cu") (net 8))
 (segment (start 85.274 70.9865) (end 85.274 63.84275) (width 0.25) (layer "B.Cu") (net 8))
 (segment (start 94.654767 67.587733) (end 94.654767 68.97909) (width 0.25) (layer "B.Cu") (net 33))
 (segment (start 94.654767 68.97909) (end 92.374495 71.259362) (width 0.25) (layer "B.Cu") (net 33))
 (segment (start 92.374495 71.259362) (end 87.446875 71.259362) (width 0.25) (layer "B.Cu") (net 33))
 (segment (start 98.186875 64.055625) (end 94.654767 67.587733) (width 0.25) (layer "B.Cu") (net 33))
 (segment (start 87.446875 73.259362) (end 86.271242 73.259362) (width 0.25) (layer "B.Cu") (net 11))
 (segment (start 80.406875 67.394995) (end 80.406875 66.595625) (width 0.25) (layer "B.Cu") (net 11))
 (segment (start 86.271242 73.259362) (end 80.406875 67.394995) (width 0.25) (layer "B.Cu") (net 11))
 (segment (start 98.186875 79.295625) (end 98.186875 78.541546) (width 0.25) (layer "B.Cu") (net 27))
 (segment (start 94.404691 74.759362) (end 87.446875 74.759362) (width 0.25) (layer "B.Cu") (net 27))
 (segment (start 98.186875 78.541546) (end 94.404691 74.759362) (width 0.25) (layer "B.Cu") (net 27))
 (segment (start 98.186875 71.675625) (end 96.103138 73.759362) (width 0.25) (layer "B.Cu") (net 30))
 (segment (start 96.103138 73.759362) (end 87.446875 73.759362) (width 0.25) (layer "B.Cu") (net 30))
 (segment (start 98.186875 76.755625) (end 95.690612 74.259362) (width 0.25) (layer "B.Cu") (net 28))
 (segment (start 95.690612 74.259362) (end 87.446875 74.259362) (width 0.25) (layer "B.Cu") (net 28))
 (segment (start 93.464141 77.486818) (end 92.236685 76.259362) (width 0.25) (layer "B.Cu") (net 23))
 (segment (start 92.236685 76.259362) (end 87.446875 76.259362) (width 0.25) (layer "B.Cu") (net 23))
 (segment (start 98.186875 89.455625) (end 93.464141 84.732891) (width 0.25) (layer "B.Cu") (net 23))
 (segment (start 93.464141 84.732891) (end 93.464141 77.486818) (width 0.25) (layer "B.Cu") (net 23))
 (segment (start 92.098875 76.759362) (end 87.446875 76.759362) (width 0.25) (layer "B.Cu") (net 22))
 (segment (start 92.868828 86.677578) (end 92.868828 77.529315) (width 0.25) (layer "B.Cu") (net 22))
 (segment (start 98.186875 91.995625) (end 92.868828 86.677578) (width 0.25) (layer "B.Cu") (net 22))
 (segment (start 92.868828 77.529315) (end 92.098875 76.759362) (width 0.25) (layer "B.Cu") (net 22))
 (segment (start 81.910612 78.259362) (end 87.446875 78.259362) (width 0.25) (layer "B.Cu") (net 15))
 (segment (start 80.406875 76.755625) (end 81.910612 78.259362) (width 0.25) (layer "B.Cu") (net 15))
 (segment (start 86.679496 77.259362) (end 83.34375 73.923616) (width 0.25) (layer "B.Cu") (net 12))
 (segment (start 87.446875 77.259362) (end 86.679496 77.259362) (width 0.25) (layer "B.Cu") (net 12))
 (segment (start 83.34375 72.0725) (end 80.406875 69.135625) (width 0.25) (layer "B.Cu") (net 12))
 (segment (start 83.34375 73.923616) (end 83.34375 72.0725) (width 0.25) (layer "B.Cu") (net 12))
 (segment (start 83.34375 83.410487) (end 83.34375 86.51875) (width 0.25) (layer "B.Cu") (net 20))
 (segment (start 87.446875 80.259362) (end 86.494875 80.259362) (width 0.25) (layer "B.Cu") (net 20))
 (segment (start 83.34375 86.51875) (end 80.406875 89.455625) (width 0.25) (layer "B.Cu") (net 20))
 (segment (start 86.494875 80.259362) (end 83.34375 83.410487) (width 0.25) (layer "B.Cu") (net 20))
 (segment (start 87.446875 84.955625) (end 80.406875 91.995625) (width 0.25) (layer "B.Cu") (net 21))
 (segment (start 87.446875 80.759362) (end 87.446875 84.955625) (width 0.25) (layer "B.Cu") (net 21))
 (segment (start 80.943138 78.759362) (end 87.446875 78.759362) (width 0.25) (layer "B.Cu") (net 16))
 (segment (start 80.406875 79.295625) (end 80.943138 78.759362) (width 0.25) (layer "B.Cu") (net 16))
 (segment (start 82.983138 79.259362) (end 87.446875 79.259362) (width 0.25) (layer "B.Cu") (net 17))
 (segment (start 80.406875 81.835625) (end 82.983138 79.259362) (width 0.25) (layer "B.Cu") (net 17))
 (segment (start 80.406875 71.675625) (end 80.406875 71.809172) (width 0.25) (layer "B.Cu") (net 13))
 (segment (start 80.406875 71.809172) (end 86.357065 77.759362) (width 0.25) (layer "B.Cu") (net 13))
 (segment (start 86.357065 77.759362) (end 87.446875 77.759362) (width 0.25) (layer "B.Cu") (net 13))
 (segment (start 80.406875 84.375625) (end 85.023138 79.759362) (width 0.25) (layer "B.Cu") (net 18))
 (segment (start 85.023138 79.759362) (end 87.446875 79.759362) (width 0.25) (layer "B.Cu") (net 18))
 (segment (start 80.406875 43.735625) (end 81.582875 42.559625) (width 0.25) (layer "F.Cu") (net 2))
 (segment (start 101.644366 45.53) (end 105.984375 45.53) (width 0.25) (layer "F.Cu") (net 2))
 (segment (start 98.673991 42.559625) (end 101.644366 45.53) (width 0.25) (layer "F.Cu") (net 2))
 (segment (start 81.582875 42.559625) (end 98.673991 42.559625) (width 0.25) (layer "F.Cu") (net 2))
 (segment (start 81.770875 44.911625) (end 80.406875 46.275625) (width 0.25) (layer "F.Cu") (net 3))
 (segment (start 100.388181 44.911625) (end 81.770875 44.911625) (width 0.25) (layer "F.Cu") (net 3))
 (segment (start 104.006556 48.53) (end 100.388181 44.911625) (width 0.25) (layer "F.Cu") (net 3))
 (segment (start 105.984375 48.53) (end 104.006556 48.53) (width 0.25) (layer "F.Cu") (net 3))
 (segment (start 111.16875 47.694918) (end 111.16875 51.196918) (width 0.25) (layer "B.Cu") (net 6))
 (segment (start 89.202875 45.099625) (end 80.72578 53.57672) (width 0.25) (layer "B.Cu") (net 6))
 (segment (start 105.49726 43.954) (end 107.427832 43.954) (width 0.25) (layer "B.Cu") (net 6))
 (segment (start 107.427832 43.954) (end 111.16875 47.694918) (width 0.25) (layer "B.Cu") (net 6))
 (segment (start 104.351635 45.099625) (end 105.49726 43.954) (width 0.25) (layer "B.Cu") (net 6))
 (segment (start 104.351635 45.099625) (end 89.202875 45.099625) (width 0.25) (layer "B.Cu") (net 6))
 (segment (start 99.392125 60.151625) (end 97.010875 60.151625) (width 0.25) (layer "F.Cu") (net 26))
 (segment (start 99.981897 66.727531) (end 99.981897 80.040603) (width 0.25) (layer "F.Cu") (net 26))
 (segment (start 117.871974 51.633483) (end 119.007974 52.769483) (width 0.25) (layer "F.Cu") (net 26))
 (segment (start 97.699759 65.419625) (end 98.673991 65.419625) (width 0.25) (layer "F.Cu") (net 26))
 (segment (start 117.578004 56.253246) (end 116.430021 56.253246) (width 0.25) (layer "F.Cu") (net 26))
 (segment (start 116.430021 56.253246) (end 114.342593 58.340674) (width 0.25) (layer "F.Cu") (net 26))
 (segment (start 99.981897 80.040603) (end 98.186875 81.835625) (width 0.25) (layer "F.Cu") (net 26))
 (segment (start 96.440625 64.160491) (end 97.699759 65.419625) (width 0.25) (layer "F.Cu") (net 26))
 (segment (start 98.673991 65.419625) (end 99.981897 66.727531) (width 0.25) (layer "F.Cu") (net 26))
 (segment (start 114.342593 58.340674) (end 101.203076 58.340674) (width 0.25) (layer "F.Cu") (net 26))
 (segment (start 97.010875 60.151625) (end 96.440625 60.721875) (width 0.25) (layer "F.Cu") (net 26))
 (segment (start 96.440625 60.721875) (end 96.440625 64.160491) (width 0.25) (layer "F.Cu") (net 26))
 (segment (start 101.203076 58.340674) (end 99.392125 60.151625) (width 0.25) (layer "F.Cu") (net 26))
 (segment (start 119.007974 54.823276) (end 117.578004 56.253246) (width 0.25) (layer "F.Cu") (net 26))
 (segment (start 119.007974 52.769483) (end 119.007974 54.823276) (width 0.25) (layer "F.Cu") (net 26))
 (segment (start 95.25008 78.89883) (end 95.25008 77.242714) (width 0.25) (layer "B.Cu") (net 26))
 (segment (start 109.228125 54.76875) (end 109.228125 55.69375) (width 0.25) (layer "B.Cu") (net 26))
 (segment (start 98.186875 81.347362) (end 98.186875 81.835625) (width 0.25) (layer "B.Cu") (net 26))
 (segment (start 109.228125 55.69375) (end 110.31775 56.783375) (width 0.25) (layer "B.Cu") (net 26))
 (segment (start 116.868629 56.783375) (end 119.007974 54.64403) (width 0.25) (layer "B.Cu") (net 26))
 (segment (start 119.007974 52.769483) (end 117.871974 51.633483) (width 0.25) (layer "B.Cu") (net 26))
 (segment (start 98.186875 81.835625) (end 95.25008 78.89883) (width 0.25) (layer "B.Cu") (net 26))
 (segment (start 95.25008 77.242714) (end 93.266728 75.259362) (width 0.25) (layer "B.Cu") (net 26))
 (segment (start 93.266728 75.259362) (end 87.446875 75.259362) (width 0.25) (layer "B.Cu") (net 26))
 (segment (start 119.007974 54.64403) (end 119.007974 52.769483) (width 0.25) (layer "B.Cu") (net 26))
 (segment (start 110.31775 56.783375) (end 116.868629 56.783375) (width 0.25) (layer "B.Cu") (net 26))
 (segment (start 96.981625 57.799625) (end 112.250552 57.799625) (width 0.25) (layer "F.Cu") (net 25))
 (segment (start 95.25 59.53125) (end 96.981625 57.799625) (width 0.25) (layer "F.Cu") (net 25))
 (segment (start 95.25 81.43875) (end 95.25 59.53125) (width 0.25) (layer "F.Cu") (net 25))
 (segment (start 112.250552 57.799625) (end 115.876694 54.173483) (width 0.25) (layer "F.Cu") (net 25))
 (segment (start 115.876694 54.173483) (end 117.871974 54.173483) (width 0.25) (layer "F.Cu") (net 25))
 (segment (start 98.186875 84.375625) (end 95.25 81.43875) (width 0.25) (layer "F.Cu") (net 25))
 (segment (start 110.228125 55.69375) (end 110.49375 55.959375) (width 0.25) (layer "B.Cu") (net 25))
 (segment (start 110.228125 54.76875) (end 110.228125 55.69375) (width 0.25) (layer "B.Cu") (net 25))
 (segment (start 116.086082 55.959375) (end 117.871974 54.173483) (width 0.25) (layer "B.Cu") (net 25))
 (segment (start 94.059454 77.444321) (end 92.374495 75.759362) (width 0.25) (layer "B.Cu") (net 25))
 (segment (start 94.059454 80.248204) (end 94.059454 77.444321) (width 0.25) (layer "B.Cu") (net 25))
 (segment (start 92.374495 75.759362) (end 87.446875 75.759362) (width 0.25) (layer "B.Cu") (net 25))
 (segment (start 98.186875 84.375625) (end 94.059454 80.248204) (width 0.25) (layer "B.Cu") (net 25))
 (segment (start 110.49375 55.959375) (end 116.086082 55.959375) (width 0.25) (layer "B.Cu") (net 25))
 (segment (start 111.66875 51.196918) (end 111.66875 47.557108) (width 0.25) (layer "B.Cu") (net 7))
 (segment (start 79.207258 42.831907) (end 79.207258 55.236008) (width 0.25) (layer "B.Cu") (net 7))
 (segment (start 111.66875 47.557108) (end 106.51256 42.400918) (width 0.25) (layer "B.Cu") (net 7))
 (segment (start 106.51256 42.400918) (end 79.638247 42.400918) (width 0.25) (layer "B.Cu") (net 7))
 (segment (start 79.638247 42.400918) (end 79.207258 42.831907) (width 0.25) (layer "B.Cu") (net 7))
 (segment (start 79.207258 55.236008) (end 80.406875 56.435625) (width 0.25) (layer "B.Cu") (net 7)))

